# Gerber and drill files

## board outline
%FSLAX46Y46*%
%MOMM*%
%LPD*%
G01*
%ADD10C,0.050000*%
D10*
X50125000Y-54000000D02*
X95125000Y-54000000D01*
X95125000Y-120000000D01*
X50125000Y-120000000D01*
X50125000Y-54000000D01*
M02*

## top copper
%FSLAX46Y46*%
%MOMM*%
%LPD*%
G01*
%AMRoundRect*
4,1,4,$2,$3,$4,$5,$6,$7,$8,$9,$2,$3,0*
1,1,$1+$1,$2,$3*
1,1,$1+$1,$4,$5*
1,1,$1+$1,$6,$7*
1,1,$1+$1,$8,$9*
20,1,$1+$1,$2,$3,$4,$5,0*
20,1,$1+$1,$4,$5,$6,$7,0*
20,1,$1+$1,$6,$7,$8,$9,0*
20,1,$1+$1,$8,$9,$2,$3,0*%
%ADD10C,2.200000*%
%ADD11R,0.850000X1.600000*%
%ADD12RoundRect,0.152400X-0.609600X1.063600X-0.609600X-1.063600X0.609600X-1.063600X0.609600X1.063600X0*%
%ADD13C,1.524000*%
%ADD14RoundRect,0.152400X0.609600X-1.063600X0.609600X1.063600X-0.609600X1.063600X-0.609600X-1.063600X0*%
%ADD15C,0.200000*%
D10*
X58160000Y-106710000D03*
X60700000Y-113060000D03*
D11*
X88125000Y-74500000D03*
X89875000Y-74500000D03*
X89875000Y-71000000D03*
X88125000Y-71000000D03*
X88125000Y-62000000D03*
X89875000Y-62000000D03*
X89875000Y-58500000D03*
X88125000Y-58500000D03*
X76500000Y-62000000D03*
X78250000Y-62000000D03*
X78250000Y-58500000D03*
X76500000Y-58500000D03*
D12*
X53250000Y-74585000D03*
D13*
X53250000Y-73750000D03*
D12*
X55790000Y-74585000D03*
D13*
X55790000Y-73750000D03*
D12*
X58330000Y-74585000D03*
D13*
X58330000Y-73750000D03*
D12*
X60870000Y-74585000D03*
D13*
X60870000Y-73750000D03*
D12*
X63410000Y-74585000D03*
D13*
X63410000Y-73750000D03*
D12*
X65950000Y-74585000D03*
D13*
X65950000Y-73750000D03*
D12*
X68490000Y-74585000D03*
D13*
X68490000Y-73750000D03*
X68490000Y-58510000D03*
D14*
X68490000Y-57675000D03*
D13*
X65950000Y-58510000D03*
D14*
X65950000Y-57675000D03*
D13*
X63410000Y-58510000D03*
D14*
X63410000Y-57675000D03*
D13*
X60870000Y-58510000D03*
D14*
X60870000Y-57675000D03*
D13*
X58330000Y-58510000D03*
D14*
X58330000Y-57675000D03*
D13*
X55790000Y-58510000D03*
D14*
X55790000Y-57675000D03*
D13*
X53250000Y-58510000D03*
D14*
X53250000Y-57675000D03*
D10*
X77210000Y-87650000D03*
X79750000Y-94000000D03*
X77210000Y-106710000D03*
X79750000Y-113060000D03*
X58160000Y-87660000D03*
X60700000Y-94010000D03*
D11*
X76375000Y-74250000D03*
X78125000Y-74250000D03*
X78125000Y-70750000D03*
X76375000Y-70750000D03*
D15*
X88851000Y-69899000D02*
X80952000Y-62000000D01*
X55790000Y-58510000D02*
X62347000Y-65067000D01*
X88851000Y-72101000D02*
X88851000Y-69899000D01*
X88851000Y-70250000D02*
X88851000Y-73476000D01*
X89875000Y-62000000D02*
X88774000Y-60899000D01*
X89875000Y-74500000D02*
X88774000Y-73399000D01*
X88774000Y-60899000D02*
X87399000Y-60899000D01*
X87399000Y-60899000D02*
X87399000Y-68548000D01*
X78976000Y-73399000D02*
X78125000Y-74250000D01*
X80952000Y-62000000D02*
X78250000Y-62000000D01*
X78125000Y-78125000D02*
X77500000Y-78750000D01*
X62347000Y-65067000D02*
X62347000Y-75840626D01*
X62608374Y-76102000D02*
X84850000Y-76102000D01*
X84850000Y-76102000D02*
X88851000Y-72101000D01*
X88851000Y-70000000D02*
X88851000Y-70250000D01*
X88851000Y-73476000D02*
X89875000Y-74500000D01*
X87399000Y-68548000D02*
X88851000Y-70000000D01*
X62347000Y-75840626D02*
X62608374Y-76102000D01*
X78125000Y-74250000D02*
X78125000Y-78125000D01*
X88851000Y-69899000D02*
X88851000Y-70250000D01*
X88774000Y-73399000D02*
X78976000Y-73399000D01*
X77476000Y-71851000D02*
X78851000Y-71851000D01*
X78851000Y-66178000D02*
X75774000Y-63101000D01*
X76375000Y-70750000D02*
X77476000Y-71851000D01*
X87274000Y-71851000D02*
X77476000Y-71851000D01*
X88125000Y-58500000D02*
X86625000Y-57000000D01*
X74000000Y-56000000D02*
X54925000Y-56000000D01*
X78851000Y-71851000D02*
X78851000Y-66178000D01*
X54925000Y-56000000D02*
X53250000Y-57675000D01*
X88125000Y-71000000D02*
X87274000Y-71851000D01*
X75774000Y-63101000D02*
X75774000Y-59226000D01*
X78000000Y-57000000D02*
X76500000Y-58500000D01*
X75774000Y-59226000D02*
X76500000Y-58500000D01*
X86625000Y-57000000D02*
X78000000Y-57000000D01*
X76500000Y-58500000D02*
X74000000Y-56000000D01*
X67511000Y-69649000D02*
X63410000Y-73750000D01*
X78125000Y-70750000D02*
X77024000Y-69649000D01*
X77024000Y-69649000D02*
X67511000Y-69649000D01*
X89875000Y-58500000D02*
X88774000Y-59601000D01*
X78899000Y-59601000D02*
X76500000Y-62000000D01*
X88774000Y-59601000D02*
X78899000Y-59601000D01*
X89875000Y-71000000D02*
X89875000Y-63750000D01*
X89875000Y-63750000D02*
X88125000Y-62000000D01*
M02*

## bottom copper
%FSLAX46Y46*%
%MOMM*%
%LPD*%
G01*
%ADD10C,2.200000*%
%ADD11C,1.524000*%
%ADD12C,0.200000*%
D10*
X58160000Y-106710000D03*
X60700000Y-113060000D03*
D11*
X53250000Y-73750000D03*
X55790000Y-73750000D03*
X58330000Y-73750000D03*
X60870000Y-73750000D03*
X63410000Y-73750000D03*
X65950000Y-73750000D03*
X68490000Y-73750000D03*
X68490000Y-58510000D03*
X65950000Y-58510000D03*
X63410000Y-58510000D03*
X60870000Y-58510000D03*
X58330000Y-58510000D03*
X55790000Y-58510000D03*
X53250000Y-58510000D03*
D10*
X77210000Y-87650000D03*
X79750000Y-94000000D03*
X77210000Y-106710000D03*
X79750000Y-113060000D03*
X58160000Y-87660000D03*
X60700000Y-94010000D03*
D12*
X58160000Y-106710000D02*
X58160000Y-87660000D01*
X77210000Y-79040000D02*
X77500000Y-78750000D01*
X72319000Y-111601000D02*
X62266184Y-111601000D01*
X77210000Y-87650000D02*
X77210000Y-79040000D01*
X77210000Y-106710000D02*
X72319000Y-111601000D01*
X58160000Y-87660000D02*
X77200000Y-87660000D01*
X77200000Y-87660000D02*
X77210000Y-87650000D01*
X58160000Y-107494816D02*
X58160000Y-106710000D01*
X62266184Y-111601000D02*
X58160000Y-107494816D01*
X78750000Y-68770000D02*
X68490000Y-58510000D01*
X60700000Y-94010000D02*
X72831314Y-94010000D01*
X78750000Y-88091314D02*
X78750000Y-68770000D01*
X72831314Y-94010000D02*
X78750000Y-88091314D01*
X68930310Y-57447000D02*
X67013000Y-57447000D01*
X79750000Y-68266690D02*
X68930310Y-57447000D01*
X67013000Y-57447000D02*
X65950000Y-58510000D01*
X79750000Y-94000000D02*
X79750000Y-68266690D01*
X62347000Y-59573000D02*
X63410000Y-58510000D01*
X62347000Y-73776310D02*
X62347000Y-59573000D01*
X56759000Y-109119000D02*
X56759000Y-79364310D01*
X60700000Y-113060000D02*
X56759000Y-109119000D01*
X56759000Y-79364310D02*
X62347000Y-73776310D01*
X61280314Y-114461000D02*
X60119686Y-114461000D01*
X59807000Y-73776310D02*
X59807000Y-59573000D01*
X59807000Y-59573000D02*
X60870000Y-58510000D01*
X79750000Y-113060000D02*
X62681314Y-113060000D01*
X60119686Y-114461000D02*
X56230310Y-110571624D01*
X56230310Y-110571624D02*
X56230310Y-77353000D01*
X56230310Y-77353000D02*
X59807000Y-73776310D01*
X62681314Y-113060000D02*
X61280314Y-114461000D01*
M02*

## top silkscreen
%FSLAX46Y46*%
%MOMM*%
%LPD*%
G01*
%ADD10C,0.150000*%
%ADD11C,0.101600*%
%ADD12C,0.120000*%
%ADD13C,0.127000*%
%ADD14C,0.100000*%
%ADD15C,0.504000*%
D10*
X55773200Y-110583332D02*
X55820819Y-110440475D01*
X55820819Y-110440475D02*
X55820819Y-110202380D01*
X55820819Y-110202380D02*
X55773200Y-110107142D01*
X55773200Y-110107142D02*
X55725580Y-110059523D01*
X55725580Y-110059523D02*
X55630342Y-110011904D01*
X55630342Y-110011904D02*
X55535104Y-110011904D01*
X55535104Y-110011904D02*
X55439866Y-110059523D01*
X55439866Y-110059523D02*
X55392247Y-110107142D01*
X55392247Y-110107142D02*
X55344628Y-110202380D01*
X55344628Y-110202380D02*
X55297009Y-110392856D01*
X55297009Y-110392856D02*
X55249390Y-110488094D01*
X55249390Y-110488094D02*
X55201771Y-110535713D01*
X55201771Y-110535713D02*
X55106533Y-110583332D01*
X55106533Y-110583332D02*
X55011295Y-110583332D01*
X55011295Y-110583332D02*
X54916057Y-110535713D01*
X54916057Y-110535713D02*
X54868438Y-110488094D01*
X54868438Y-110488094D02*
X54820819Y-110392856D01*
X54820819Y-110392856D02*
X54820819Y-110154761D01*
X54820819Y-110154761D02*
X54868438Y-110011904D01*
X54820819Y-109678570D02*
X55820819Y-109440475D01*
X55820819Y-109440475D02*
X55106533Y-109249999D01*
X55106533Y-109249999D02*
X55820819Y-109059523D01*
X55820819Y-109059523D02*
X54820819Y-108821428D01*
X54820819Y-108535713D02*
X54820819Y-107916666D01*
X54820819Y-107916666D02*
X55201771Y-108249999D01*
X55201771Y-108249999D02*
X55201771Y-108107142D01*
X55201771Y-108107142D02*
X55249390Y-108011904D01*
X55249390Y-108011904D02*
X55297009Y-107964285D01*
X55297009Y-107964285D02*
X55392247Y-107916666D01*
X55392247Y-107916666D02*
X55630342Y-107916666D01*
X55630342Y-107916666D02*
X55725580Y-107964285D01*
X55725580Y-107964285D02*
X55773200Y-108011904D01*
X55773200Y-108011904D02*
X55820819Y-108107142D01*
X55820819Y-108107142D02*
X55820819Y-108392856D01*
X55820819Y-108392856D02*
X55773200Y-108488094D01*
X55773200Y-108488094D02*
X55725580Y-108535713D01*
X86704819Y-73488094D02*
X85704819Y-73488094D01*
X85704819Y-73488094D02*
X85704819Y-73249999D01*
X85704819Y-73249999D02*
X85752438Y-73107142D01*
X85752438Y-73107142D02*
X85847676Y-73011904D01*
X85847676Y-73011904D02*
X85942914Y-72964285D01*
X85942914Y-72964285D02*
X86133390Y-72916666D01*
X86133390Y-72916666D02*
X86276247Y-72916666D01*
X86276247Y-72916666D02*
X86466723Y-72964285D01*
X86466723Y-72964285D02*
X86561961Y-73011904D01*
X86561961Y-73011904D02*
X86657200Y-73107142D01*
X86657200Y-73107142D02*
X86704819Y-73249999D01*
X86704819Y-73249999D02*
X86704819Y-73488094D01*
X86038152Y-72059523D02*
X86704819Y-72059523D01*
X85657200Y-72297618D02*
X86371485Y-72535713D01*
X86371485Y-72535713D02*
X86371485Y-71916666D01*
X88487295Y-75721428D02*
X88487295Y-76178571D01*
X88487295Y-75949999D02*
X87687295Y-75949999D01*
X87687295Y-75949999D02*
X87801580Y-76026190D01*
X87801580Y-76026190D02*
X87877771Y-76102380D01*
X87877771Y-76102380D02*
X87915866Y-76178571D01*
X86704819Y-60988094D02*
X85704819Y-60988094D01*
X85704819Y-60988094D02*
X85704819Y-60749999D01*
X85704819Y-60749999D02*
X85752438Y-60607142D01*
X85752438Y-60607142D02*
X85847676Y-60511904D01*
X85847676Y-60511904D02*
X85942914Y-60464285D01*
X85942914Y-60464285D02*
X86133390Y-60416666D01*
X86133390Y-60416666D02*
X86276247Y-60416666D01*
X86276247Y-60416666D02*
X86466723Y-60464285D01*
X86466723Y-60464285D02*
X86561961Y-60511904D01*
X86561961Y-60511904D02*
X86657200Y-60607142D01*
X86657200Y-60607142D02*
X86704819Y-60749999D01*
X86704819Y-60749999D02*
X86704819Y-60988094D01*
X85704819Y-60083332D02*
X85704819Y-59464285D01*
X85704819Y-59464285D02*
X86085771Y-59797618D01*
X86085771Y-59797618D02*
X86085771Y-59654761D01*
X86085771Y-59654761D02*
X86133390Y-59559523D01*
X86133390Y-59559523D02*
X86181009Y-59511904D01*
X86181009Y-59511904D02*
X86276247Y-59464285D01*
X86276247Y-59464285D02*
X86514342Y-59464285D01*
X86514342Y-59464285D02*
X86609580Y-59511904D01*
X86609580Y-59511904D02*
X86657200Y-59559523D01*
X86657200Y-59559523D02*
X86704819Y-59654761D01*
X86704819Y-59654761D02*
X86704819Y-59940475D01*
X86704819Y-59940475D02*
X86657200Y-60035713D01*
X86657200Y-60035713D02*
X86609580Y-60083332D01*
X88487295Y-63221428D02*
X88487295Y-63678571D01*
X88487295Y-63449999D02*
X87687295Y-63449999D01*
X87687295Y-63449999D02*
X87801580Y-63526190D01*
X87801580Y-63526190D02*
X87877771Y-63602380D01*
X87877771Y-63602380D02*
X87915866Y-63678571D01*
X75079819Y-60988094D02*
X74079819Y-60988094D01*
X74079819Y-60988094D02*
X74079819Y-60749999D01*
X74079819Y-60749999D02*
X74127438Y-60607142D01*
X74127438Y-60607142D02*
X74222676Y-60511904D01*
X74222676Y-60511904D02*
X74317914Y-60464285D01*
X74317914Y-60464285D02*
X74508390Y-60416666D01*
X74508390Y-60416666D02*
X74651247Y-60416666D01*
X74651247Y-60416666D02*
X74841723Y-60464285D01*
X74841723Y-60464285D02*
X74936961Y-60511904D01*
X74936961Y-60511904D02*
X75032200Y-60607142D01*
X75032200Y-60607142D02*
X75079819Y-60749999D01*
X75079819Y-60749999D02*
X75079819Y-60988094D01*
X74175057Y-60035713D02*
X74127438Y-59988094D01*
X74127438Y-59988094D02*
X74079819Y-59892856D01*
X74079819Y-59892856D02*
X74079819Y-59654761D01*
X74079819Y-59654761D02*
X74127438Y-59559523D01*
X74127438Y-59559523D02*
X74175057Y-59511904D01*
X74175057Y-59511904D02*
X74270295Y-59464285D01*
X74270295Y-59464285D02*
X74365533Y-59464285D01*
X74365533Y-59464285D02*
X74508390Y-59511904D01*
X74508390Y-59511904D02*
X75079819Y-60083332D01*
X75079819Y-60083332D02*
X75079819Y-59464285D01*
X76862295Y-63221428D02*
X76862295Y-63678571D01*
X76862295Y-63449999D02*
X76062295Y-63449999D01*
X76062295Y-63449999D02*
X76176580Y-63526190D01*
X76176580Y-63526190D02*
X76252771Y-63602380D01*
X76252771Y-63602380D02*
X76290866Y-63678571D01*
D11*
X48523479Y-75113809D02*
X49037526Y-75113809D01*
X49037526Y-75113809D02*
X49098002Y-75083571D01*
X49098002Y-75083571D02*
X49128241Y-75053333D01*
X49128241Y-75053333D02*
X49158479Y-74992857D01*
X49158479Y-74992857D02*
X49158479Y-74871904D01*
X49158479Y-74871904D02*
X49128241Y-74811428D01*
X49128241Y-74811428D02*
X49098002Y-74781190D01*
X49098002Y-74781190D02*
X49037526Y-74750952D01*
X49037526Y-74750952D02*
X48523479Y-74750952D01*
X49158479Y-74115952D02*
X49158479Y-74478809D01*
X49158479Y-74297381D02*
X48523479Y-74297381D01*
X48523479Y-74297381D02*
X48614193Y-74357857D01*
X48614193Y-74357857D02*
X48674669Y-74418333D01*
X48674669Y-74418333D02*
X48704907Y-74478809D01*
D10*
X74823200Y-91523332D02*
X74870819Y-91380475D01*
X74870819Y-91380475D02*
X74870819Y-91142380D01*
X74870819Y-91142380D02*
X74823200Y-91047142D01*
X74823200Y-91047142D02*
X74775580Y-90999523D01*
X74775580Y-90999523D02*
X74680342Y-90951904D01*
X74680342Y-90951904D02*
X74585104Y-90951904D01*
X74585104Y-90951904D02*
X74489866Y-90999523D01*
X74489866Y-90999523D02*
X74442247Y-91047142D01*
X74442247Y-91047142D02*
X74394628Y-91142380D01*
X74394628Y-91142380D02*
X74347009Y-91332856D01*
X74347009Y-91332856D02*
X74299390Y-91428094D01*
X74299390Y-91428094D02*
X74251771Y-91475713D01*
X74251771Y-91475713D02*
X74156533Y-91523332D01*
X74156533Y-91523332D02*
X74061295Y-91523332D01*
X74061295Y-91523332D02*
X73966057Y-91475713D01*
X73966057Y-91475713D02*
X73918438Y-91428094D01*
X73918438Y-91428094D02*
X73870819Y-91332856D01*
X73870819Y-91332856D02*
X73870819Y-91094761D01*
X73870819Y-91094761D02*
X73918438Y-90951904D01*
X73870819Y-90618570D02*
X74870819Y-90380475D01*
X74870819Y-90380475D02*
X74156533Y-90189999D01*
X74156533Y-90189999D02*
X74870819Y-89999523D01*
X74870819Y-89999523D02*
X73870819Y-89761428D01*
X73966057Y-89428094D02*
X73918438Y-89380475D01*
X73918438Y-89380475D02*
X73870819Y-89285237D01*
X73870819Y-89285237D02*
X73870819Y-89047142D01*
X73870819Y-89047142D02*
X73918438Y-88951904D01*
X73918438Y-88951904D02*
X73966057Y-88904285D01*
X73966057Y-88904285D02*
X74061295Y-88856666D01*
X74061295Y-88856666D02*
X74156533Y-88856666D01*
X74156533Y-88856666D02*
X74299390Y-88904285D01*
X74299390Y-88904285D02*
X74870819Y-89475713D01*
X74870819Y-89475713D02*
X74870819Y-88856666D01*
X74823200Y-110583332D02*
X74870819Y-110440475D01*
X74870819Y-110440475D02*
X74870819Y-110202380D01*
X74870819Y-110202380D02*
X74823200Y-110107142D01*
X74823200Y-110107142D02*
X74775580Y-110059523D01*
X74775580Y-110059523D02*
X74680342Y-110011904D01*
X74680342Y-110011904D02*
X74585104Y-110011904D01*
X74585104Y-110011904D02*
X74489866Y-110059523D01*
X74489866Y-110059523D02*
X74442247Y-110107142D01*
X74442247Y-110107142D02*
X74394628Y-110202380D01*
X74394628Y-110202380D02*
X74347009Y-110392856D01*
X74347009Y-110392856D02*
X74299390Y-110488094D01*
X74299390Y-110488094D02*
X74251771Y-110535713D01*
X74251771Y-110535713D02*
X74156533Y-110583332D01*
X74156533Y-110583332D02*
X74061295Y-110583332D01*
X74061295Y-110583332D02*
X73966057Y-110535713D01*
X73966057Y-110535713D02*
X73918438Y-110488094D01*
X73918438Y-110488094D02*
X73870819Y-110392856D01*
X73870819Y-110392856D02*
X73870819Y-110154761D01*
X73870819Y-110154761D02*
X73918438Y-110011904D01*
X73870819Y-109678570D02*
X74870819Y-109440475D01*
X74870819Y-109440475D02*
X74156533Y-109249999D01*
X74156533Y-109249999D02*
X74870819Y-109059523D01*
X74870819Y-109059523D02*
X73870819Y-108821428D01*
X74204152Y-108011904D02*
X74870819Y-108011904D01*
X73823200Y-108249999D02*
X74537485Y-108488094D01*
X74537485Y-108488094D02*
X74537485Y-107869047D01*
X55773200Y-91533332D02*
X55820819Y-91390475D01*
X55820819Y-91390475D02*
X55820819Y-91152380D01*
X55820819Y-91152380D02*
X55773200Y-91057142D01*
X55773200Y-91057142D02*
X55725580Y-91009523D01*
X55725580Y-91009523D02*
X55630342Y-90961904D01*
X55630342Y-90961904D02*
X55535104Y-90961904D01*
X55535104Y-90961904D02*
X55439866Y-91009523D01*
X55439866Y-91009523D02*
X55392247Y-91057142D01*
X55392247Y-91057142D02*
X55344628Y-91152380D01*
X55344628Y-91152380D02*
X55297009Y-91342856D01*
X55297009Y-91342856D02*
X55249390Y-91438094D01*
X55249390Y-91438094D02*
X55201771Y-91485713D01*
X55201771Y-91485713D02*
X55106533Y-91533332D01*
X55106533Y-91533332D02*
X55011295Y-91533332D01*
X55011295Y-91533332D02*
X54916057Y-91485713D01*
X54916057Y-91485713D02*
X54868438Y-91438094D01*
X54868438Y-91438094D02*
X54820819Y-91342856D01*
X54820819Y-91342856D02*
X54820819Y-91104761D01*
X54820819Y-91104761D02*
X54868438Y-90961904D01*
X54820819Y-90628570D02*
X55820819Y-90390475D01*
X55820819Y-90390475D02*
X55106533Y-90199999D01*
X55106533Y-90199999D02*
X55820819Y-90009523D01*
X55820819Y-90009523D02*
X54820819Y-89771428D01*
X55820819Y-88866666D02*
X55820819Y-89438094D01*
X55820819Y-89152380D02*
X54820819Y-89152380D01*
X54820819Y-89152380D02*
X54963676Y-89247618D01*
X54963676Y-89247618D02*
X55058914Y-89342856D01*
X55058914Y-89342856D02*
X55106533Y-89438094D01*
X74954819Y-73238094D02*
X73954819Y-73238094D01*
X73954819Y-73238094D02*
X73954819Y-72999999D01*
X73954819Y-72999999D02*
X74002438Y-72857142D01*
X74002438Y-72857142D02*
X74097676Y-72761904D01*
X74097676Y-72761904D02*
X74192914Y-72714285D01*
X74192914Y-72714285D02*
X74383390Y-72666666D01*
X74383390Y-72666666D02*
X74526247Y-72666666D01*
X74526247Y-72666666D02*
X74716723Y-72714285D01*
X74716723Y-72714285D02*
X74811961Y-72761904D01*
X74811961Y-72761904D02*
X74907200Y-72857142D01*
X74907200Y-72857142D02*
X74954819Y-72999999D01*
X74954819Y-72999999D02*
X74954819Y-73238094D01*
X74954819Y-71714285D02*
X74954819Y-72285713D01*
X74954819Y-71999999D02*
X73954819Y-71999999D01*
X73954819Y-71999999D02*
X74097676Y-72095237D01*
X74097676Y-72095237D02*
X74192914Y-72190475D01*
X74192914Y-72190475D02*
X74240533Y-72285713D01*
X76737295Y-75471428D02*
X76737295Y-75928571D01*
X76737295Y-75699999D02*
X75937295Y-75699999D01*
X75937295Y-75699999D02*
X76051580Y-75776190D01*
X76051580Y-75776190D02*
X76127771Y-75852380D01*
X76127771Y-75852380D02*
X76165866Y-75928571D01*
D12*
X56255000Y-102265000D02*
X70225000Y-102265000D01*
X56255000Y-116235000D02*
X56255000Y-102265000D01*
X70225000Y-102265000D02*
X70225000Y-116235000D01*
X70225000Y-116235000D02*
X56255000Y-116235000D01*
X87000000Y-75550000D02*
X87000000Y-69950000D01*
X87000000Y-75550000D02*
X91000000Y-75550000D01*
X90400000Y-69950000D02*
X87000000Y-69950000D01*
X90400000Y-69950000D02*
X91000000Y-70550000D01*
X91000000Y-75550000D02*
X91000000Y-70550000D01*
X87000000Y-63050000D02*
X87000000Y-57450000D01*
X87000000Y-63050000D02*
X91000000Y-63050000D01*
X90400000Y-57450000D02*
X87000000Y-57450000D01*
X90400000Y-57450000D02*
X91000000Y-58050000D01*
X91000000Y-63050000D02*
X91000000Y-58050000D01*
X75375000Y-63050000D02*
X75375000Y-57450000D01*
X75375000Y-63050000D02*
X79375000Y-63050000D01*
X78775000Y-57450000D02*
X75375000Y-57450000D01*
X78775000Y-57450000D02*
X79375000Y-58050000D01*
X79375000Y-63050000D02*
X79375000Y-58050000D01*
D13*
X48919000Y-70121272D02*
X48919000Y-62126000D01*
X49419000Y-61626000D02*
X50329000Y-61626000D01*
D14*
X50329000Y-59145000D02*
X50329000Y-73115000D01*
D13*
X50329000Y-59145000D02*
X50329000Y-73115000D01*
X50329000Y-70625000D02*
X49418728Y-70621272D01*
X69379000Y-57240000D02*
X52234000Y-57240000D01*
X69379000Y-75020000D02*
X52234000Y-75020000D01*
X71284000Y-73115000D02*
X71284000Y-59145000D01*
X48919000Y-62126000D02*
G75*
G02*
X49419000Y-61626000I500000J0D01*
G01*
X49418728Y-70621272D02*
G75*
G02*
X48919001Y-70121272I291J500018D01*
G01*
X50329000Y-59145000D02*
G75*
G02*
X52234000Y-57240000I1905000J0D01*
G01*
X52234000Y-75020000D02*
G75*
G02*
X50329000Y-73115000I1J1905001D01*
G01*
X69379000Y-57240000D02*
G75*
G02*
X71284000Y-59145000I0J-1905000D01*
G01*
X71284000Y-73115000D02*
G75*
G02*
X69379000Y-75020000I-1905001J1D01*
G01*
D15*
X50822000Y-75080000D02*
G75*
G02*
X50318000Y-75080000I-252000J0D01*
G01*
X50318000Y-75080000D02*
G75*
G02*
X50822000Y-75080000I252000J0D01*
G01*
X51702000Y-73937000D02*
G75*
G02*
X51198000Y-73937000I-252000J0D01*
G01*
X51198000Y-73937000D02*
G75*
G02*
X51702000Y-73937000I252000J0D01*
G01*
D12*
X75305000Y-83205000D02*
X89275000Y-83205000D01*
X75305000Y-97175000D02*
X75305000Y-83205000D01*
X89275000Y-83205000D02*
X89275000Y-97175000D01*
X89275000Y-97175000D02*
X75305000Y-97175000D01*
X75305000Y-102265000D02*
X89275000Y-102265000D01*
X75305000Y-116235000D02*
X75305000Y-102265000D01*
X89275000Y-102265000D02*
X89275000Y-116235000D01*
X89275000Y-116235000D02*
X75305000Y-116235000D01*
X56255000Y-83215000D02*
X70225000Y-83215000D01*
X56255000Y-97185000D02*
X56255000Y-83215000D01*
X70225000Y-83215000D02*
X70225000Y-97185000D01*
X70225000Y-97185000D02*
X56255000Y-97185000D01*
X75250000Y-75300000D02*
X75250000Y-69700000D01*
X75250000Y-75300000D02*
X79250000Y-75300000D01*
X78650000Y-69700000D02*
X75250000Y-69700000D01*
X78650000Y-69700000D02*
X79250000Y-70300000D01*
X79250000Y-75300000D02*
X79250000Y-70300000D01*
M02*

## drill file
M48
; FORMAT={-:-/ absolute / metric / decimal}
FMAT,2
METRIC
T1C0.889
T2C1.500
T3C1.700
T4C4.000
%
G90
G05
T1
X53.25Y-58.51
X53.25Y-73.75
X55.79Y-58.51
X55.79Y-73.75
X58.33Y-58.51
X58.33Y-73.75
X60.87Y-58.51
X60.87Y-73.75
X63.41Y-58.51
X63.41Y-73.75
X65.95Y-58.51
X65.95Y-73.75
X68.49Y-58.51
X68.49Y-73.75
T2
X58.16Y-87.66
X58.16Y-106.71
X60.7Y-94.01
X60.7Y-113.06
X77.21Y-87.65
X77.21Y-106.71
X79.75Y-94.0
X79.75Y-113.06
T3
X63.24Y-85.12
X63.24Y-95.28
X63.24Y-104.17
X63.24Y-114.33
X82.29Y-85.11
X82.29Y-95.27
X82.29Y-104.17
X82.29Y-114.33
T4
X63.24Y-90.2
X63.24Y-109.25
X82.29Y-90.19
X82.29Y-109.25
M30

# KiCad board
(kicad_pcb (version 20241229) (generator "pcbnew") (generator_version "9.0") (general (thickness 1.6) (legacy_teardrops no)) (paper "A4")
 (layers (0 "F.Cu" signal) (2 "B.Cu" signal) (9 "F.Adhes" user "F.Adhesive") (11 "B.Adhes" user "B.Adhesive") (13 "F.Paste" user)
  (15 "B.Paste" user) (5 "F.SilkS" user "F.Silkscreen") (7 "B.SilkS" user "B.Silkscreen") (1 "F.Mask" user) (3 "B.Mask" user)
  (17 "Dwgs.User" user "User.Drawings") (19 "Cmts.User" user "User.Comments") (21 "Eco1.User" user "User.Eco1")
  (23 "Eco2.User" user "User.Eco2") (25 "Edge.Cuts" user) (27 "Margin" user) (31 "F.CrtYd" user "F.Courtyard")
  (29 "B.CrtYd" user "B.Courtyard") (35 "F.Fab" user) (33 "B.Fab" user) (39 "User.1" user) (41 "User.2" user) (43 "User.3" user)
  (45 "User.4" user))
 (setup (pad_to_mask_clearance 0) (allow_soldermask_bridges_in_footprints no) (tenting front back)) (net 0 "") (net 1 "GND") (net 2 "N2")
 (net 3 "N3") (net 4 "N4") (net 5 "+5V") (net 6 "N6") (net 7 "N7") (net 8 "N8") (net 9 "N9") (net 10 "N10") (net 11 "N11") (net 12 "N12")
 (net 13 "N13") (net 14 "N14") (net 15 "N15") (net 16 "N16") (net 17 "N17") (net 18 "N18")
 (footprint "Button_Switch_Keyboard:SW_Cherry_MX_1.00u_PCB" (layer "F.Cu") (at 58.16 106.71 90)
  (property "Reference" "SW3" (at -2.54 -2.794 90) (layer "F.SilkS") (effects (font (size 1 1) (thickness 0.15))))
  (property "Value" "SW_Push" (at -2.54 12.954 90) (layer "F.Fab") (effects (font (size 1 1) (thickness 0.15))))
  (fp_line (start 4.445 -1.905) (end 4.445 12.065) (stroke (width 0.12) (type solid)) (layer "F.SilkS"))
  (fp_line (start -9.525 -1.905) (end 4.445 -1.905) (stroke (width 0.12) (type solid)) (layer "F.SilkS"))
  (fp_line (start 4.445 12.065) (end -9.525 12.065) (stroke (width 0.12) (type solid)) (layer "F.SilkS"))
  (fp_line (start -9.525 12.065) (end -9.525 -1.905) (stroke (width 0.12) (type solid)) (layer "F.SilkS"))
  (pad "" np_thru_hole circle (at -7.62 5.08 90) (size 1.7 1.7) (drill 1.7) (layers "*.Cu" "*.Mask"))
  (pad "" np_thru_hole circle (at -2.54 5.08 90) (size 4 4) (drill 4) (layers "*.Cu" "*.Mask"))
  (pad "" np_thru_hole circle (at 2.54 5.08 90) (size 1.7 1.7) (drill 1.7) (layers "*.Cu" "*.Mask"))
  (pad "1" thru_hole circle (at 0 0 90) (size 2.2 2.2) (drill 1.5) (layers "*.Cu" "*.Mask") (remove_unused_layers no) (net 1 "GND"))
  (pad "2" thru_hole circle (at -6.35 2.54 90) (size 2.2 2.2) (drill 1.5) (layers "*.Cu" "*.Mask") (remove_unused_layers no) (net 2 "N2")))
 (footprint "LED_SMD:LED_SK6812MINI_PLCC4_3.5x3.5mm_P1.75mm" (layer "F.Cu") (at 89 72.75 90)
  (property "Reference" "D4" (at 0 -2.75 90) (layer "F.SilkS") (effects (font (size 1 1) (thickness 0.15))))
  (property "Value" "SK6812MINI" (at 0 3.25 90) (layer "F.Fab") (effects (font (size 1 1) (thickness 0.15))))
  (fp_line (start -2.8 -2) (end 2.8 -2) (stroke (width 0.12) (type solid)) (layer "F.SilkS"))
  (fp_line (start -2.8 -2) (end -2.8 2) (stroke (width 0.12) (type default)) (layer "F.SilkS"))
  (fp_line (start 2.8 1.4) (end 2.8 -2) (stroke (width 0.12) (type solid)) (layer "F.SilkS"))
  (fp_line (start 2.8 1.4) (end 2.2 2) (stroke (width 0.12) (type default)) (layer "F.SilkS"))
  (fp_line (start -2.8 2) (end 2.2 2) (stroke (width 0.12) (type solid)) (layer "F.SilkS"))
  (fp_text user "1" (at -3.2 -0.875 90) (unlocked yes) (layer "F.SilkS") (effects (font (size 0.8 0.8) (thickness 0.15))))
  (pad "1" smd rect (at -1.75 -0.875 90) (size 1.6 0.85) (layers "F.Cu" "F.Mask" "F.Paste") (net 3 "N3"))
  (pad "2" smd rect (at -1.75 0.875 90) (size 1.6 0.85) (layers "F.Cu" "F.Mask" "F.Paste") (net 1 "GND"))
  (pad "3" smd rect (at 1.75 0.875 90) (size 1.6 0.85) (layers "F.Cu" "F.Mask" "F.Paste") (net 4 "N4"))
  (pad "4" smd rect (at 1.75 -0.875 90) (size 1.6 0.85) (layers "F.Cu" "F.Mask" "F.Paste") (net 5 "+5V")))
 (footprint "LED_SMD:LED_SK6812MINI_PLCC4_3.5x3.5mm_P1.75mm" (layer "F.Cu") (at 89 60.25 90)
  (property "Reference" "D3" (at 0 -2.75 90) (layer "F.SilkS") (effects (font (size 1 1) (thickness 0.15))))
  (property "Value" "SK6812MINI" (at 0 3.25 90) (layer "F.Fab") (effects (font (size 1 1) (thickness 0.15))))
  (fp_line (start -2.8 -2) (end 2.8 -2) (stroke (width 0.12) (type solid)) (layer "F.SilkS"))
  (fp_line (start -2.8 -2) (end -2.8 2) (stroke (width 0.12) (type default)) (layer "F.SilkS"))
  (fp_line (start 2.8 1.4) (end 2.8 -2) (stroke (width 0.12) (type solid)) (layer "F.SilkS"))
  (fp_line (start 2.8 1.4) (end 2.2 2) (stroke (width 0.12) (type default)) (layer "F.SilkS"))
  (fp_line (start -2.8 2) (end 2.2 2) (stroke (width 0.12) (type solid)) (layer "F.SilkS"))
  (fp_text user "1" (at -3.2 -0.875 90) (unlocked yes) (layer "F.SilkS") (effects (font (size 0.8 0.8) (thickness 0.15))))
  (pad "1" smd rect (at -1.75 -0.875 90) (size 1.6 0.85) (layers "F.Cu" "F.Mask" "F.Paste") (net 4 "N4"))
  (pad "2" smd rect (at -1.75 0.875 90) (size 1.6 0.85) (layers "F.Cu" "F.Mask" "F.Paste") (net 1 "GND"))
  (pad "3" smd rect (at 1.75 0.875 90) (size 1.6 0.85) (layers "F.Cu" "F.Mask" "F.Paste") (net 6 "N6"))
  (pad "4" smd rect (at 1.75 -0.875 90) (size 1.6 0.85) (layers "F.Cu" "F.Mask" "F.Paste") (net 5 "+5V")))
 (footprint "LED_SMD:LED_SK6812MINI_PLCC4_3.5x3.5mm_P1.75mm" (layer "F.Cu") (at 77.375 60.25 90)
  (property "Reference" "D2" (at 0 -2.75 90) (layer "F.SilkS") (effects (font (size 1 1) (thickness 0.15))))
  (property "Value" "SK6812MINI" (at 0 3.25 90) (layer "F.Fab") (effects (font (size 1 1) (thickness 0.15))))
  (fp_line (start -2.8 -2) (end 2.8 -2) (stroke (width 0.12) (type solid)) (layer "F.SilkS"))
  (fp_line (start -2.8 -2) (end -2.8 2) (stroke (width 0.12) (type default)) (layer "F.SilkS"))
  (fp_line (start 2.8 1.4) (end 2.8 -2) (stroke (width 0.12) (type solid)) (layer "F.SilkS"))
  (fp_line (start 2.8 1.4) (end 2.2 2) (stroke (width 0.12) (type default)) (layer "F.SilkS"))
  (fp_line (start -2.8 2) (end 2.2 2) (stroke (width 0.12) (type solid)) (layer "F.SilkS"))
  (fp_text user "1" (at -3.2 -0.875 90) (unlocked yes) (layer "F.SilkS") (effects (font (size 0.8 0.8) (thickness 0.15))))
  (pad "1" smd rect (at -1.75 -0.875 90) (size 1.6 0.85) (layers "F.Cu" "F.Mask" "F.Paste") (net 6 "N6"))
  (pad "2" smd rect (at -1.75 0.875 90) (size 1.6 0.85) (layers "F.Cu" "F.Mask" "F.Paste") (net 1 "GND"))
  (pad "3" smd rect (at 1.75 0.875 90) (size 1.6 0.85) (layers "F.Cu" "F.Mask" "F.Paste") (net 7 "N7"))
  (pad "4" smd rect (at 1.75 -0.875 90) (size 1.6 0.85) (layers "F.Cu" "F.Mask" "F.Paste") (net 5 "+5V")))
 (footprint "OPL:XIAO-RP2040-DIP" (layer "F.Cu") (at 60.87 66.13 90)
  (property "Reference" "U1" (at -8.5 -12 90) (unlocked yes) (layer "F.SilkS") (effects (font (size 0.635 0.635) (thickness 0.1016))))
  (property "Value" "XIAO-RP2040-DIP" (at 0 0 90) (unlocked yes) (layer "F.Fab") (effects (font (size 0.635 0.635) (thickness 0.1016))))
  (fp_line (start -3.991272 -11.951) (end 4.004 -11.951) (stroke (width 0.127) (type solid)) (layer "F.SilkS"))
  (fp_line (start 4.504 -11.451) (end 4.504 -10.541) (stroke (width 0.127) (type solid)) (layer "F.SilkS"))
  (fp_line (start 6.985 -10.541) (end -6.985 -10.541) (stroke (width 0.1) (type solid)) (layer "F.SilkS"))
  (fp_line (start 6.985 -10.541) (end -6.985 -10.541) (stroke (width 0.127) (type solid)) (layer "F.SilkS"))
  (fp_line (start -4.495 -10.541) (end -4.491272 -11.451272) (stroke (width 0.127) (type solid)) (layer "F.SilkS"))
  (fp_line (start 8.89 8.509) (end 8.89 -8.636) (stroke (width 0.127) (type solid)) (layer "F.SilkS"))
  (fp_line (start -8.89 8.509) (end -8.89 -8.636) (stroke (width 0.127) (type solid)) (layer "F.SilkS"))
  (fp_line (start -6.985 10.414) (end 6.985 10.414) (stroke (width 0.127) (type solid)) (layer "F.SilkS"))
  (fp_arc (start 4.004 -11.951) (mid 4.357553 -11.804553) (end 4.504 -11.451) (stroke (width 0.127) (type default)) (layer "F.SilkS"))
  (fp_arc (start -4.491272 -11.451272) (mid -4.344728 -11.80464) (end -3.991272 -11.951) (stroke (width 0.127) (type default))
   (layer "F.SilkS"))
  (fp_arc (start 6.985 -10.541) (mid 8.332038 -9.983038) (end 8.89 -8.636) (stroke (width 0.127) (type solid)) (layer "F.SilkS"))
  (fp_arc (start -8.89 -8.636) (mid -8.332038 -9.983038) (end -6.985 -10.541) (stroke (width 0.127) (type solid)) (layer "F.SilkS"))
  (fp_arc (start 8.89 8.509) (mid 8.332038 9.856038) (end 6.985 10.414) (stroke (width 0.127) (type solid)) (layer "F.SilkS"))
  (fp_arc (start -6.985 10.414) (mid -8.332038 9.856038) (end -8.89 8.509) (stroke (width 0.127) (type solid)) (layer "F.SilkS"))
  (fp_circle (center -8.95 -10.3) (end -8.95 -10.554) (stroke (width 0.5) (type solid)) (fill yes) (layer "F.SilkS"))
  (fp_circle (center -7.807 -9.42) (end -7.807 -9.674) (stroke (width 0.5) (type solid)) (fill yes) (layer "F.SilkS"))
  (pad "1" smd roundrect (at -8.455 -7.62 270) (size 2.432 1.524) (layers "F.Cu" "F.Mask") (roundrect_rratio 0.1) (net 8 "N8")
   (thermal_bridge_angle 45))
  (pad "1" thru_hole circle (at -7.62 -7.62 270) (size 1.524 1.524) (drill 0.889) (layers "*.Cu" "*.Mask") (remove_unused_layers no)
   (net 8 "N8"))
  (pad "2" smd roundrect (at -8.455 -5.08 270) (size 2.432 1.524) (layers "F.Cu" "F.Mask") (roundrect_rratio 0.1) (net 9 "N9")
   (thermal_bridge_angle 45))
  (pad "2" thru_hole circle (at -7.62 -5.08 270) (size 1.524 1.524) (drill 0.889) (layers "*.Cu" "*.Mask") (remove_unused_layers no)
   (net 9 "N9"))
  (pad "3" smd roundrect (at -8.455 -2.54 270) (size 2.432 1.524) (layers "F.Cu" "F.Mask") (roundrect_rratio 0.1) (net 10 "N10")
   (thermal_bridge_angle 45))
  (pad "3" thru_hole circle (at -7.62 -2.54 270) (size 1.524 1.524) (drill 0.889) (layers "*.Cu" "*.Mask") (remove_unused_layers no)
   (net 10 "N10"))
  (pad "4" smd roundrect (at -8.455 0 270) (size 2.432 1.524) (layers "F.Cu" "F.Mask") (roundrect_rratio 0.1) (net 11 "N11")
   (thermal_bridge_angle 45))
  (pad "4" thru_hole circle (at -7.62 0 270) (size 1.524 1.524) (drill 0.889) (layers "*.Cu" "*.Mask") (remove_unused_layers no)
   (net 11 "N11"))
  (pad "5" smd roundrect (at -8.455 2.54 270) (size 2.432 1.524) (layers "F.Cu" "F.Mask") (roundrect_rratio 0.1) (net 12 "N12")
   (thermal_bridge_angle 45))
  (pad "5" thru_hole circle (at -7.62 2.54 270) (size 1.524 1.524) (drill 0.889) (layers "*.Cu" "*.Mask") (remove_unused_layers no)
   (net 12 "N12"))
  (pad "6" smd roundrect (at -8.455 5.08 270) (size 2.432 1.524) (layers "F.Cu" "F.Mask") (roundrect_rratio 0.1) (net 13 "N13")
   (thermal_bridge_angle 45))
  (pad "6" thru_hole circle (at -7.62 5.08 270) (size 1.524 1.524) (drill 0.889) (layers "*.Cu" "*.Mask") (remove_unused_layers no)
   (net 13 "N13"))
  (pad "7" smd roundrect (at -8.455 7.62 270) (size 2.432 1.524) (layers "F.Cu" "F.Mask") (roundrect_rratio 0.1) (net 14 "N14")
   (thermal_bridge_angle 45))
  (pad "7" thru_hole circle (at -7.62 7.62 270) (size 1.524 1.524) (drill 0.889) (layers "*.Cu" "*.Mask") (remove_unused_layers no)
   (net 14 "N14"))
  (pad "8" thru_hole circle (at 7.62 7.62 90) (size 1.524 1.524) (drill 0.889) (layers "*.Cu" "*.Mask") (remove_unused_layers no)
   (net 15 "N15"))
  (pad "8" smd roundrect (at 8.455 7.62 90) (size 2.432 1.524) (layers "F.Cu" "F.Mask") (roundrect_rratio 0.1) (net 15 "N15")
   (thermal_bridge_angle 45))
  (pad "9" thru_hole circle (at 7.62 5.08 90) (size 1.524 1.524) (drill 0.889) (layers "*.Cu" "*.Mask") (remove_unused_layers no)
   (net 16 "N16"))
  (pad "9" smd roundrect (at 8.455 5.08 90) (size 2.432 1.524) (layers "F.Cu" "F.Mask") (roundrect_rratio 0.1) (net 16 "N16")
   (thermal_bridge_angle 45))
  (pad "10" thru_hole circle (at 7.62 2.54 90) (size 1.524 1.524) (drill 0.889) (layers "*.Cu" "*.Mask") (remove_unused_layers no)
   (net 2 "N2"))
  (pad "10" smd roundrect (at 8.455 2.54 90) (size 2.432 1.524) (layers "F.Cu" "F.Mask") (roundrect_rratio 0.1) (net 2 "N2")
   (thermal_bridge_angle 45))
  (pad "11" thru_hole circle (at 7.62 0 90) (size 1.524 1.524) (drill 0.889) (layers "*.Cu" "*.Mask") (remove_unused_layers no)
   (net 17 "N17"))
  (pad "11" smd roundrect (at 8.455 0 90) (size 2.432 1.524) (layers "F.Cu" "F.Mask") (roundrect_rratio 0.1) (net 17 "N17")
   (thermal_bridge_angle 45))
  (pad "12" thru_hole circle (at 7.62 -2.54 90) (size 1.524 1.524) (drill 0.889) (layers "*.Cu" "*.Mask") (remove_unused_layers no)
   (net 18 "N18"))
  (pad "12" smd roundrect (at 8.455 -2.54 90) (size 2.432 1.524) (layers "F.Cu" "F.Mask") (roundrect_rratio 0.1) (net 18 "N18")
   (thermal_bridge_angle 45))
  (pad "13" thru_hole circle (at 7.62 -5.08 90) (size 1.524 1.524) (drill 0.889) (layers "*.Cu" "*.Mask") (remove_unused_layers no)
   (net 1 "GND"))
  (pad "13" smd roundrect (at 8.455 -5.08 90) (size 2.432 1.524) (layers "F.Cu" "F.Mask") (roundrect_rratio 0.1) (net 1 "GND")
   (thermal_bridge_angle 45))
  (pad "14" thru_hole circle (at 7.62 -7.62 90) (size 1.524 1.524) (drill 0.889) (layers "*.Cu" "*.Mask") (remove_unused_layers no)
   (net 5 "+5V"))
  (pad "14" smd roundrect (at 8.455 -7.62 90) (size 2.432 1.524) (layers "F.Cu" "F.Mask") (roundrect_rratio 0.1) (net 5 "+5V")
   (thermal_bridge_angle 45)))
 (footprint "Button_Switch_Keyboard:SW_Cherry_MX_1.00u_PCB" (layer "F.Cu") (at 77.21 87.65 90)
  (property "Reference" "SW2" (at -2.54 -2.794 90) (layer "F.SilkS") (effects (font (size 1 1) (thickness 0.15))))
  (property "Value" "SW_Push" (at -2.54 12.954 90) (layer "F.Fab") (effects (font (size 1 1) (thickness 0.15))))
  (fp_line (start 4.445 -1.905) (end 4.445 12.065) (stroke (width 0.12) (type solid)) (layer "F.SilkS"))
  (fp_line (start -9.525 -1.905) (end 4.445 -1.905) (stroke (width 0.12) (type solid)) (layer "F.SilkS"))
  (fp_line (start 4.445 12.065) (end -9.525 12.065) (stroke (width 0.12) (type solid)) (layer "F.SilkS"))
  (fp_line (start -9.525 12.065) (end -9.525 -1.905) (stroke (width 0.12) (type solid)) (layer "F.SilkS"))
  (pad "" np_thru_hole circle (at -7.62 5.08 90) (size 1.7 1.7) (drill 1.7) (layers "*.Cu" "*.Mask"))
  (pad "" np_thru_hole circle (at -2.54 5.08 90) (size 4 4) (drill 4) (layers "*.Cu" "*.Mask"))
  (pad "" np_thru_hole circle (at 2.54 5.08 90) (size 1.7 1.7) (drill 1.7) (layers "*.Cu" "*.Mask"))
  (pad "1" thru_hole circle (at 0 0 90) (size 2.2 2.2) (drill 1.5) (layers "*.Cu" "*.Mask") (remove_unused_layers no) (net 1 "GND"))
  (pad "2" thru_hole circle (at -6.35 2.54 90) (size 2.2 2.2) (drill 1.5) (layers "*.Cu" "*.Mask") (remove_unused_layers no) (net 16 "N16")))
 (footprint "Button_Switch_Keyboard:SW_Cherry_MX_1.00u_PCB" (layer "F.Cu") (at 77.21 106.71 90)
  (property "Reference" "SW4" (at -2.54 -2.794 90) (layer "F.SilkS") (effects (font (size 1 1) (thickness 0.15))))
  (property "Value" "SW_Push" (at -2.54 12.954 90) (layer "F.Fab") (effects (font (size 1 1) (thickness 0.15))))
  (fp_line (start 4.445 -1.905) (end 4.445 12.065) (stroke (width 0.12) (type solid)) (layer "F.SilkS"))
  (fp_line (start -9.525 -1.905) (end 4.445 -1.905) (stroke (width 0.12) (type solid)) (layer "F.SilkS"))
  (fp_line (start 4.445 12.065) (end -9.525 12.065) (stroke (width 0.12) (type solid)) (layer "F.SilkS"))
  (fp_line (start -9.525 12.065) (end -9.525 -1.905) (stroke (width 0.12) (type solid)) (layer "F.SilkS"))
  (pad "" np_thru_hole circle (at -7.62 5.08 90) (size 1.7 1.7) (drill 1.7) (layers "*.Cu" "*.Mask"))
  (pad "" np_thru_hole circle (at -2.54 5.08 90) (size 4 4) (drill 4) (layers "*.Cu" "*.Mask"))
  (pad "" np_thru_hole circle (at 2.54 5.08 90) (size 1.7 1.7) (drill 1.7) (layers "*.Cu" "*.Mask"))
  (pad "1" thru_hole circle (at 0 0 90) (size 2.2 2.2) (drill 1.5) (layers "*.Cu" "*.Mask") (remove_unused_layers no) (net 1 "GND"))
  (pad "2" thru_hole circle (at -6.35 2.54 90) (size 2.2 2.2) (drill 1.5) (layers "*.Cu" "*.Mask") (remove_unused_layers no) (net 17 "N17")))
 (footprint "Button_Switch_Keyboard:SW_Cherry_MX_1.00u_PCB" (layer "F.Cu") (at 58.16 87.66 90)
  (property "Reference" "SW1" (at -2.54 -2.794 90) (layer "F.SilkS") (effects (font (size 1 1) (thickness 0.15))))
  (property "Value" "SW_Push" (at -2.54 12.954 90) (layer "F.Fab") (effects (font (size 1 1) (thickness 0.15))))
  (fp_line (start 4.445 -1.905) (end 4.445 12.065) (stroke (width 0.12) (type solid)) (layer "F.SilkS"))
  (fp_line (start -9.525 -1.905) (end 4.445 -1.905) (stroke (width 0.12) (type solid)) (layer "F.SilkS"))
  (fp_line (start 4.445 12.065) (end -9.525 12.065) (stroke (width 0.12) (type solid)) (layer "F.SilkS"))
  (fp_line (start -9.525 12.065) (end -9.525 -1.905) (stroke (width 0.12) (type solid)) (layer "F.SilkS"))
  (pad "" np_thru_hole circle (at -7.62 5.08 90) (size 1.7 1.7) (drill 1.7) (layers "*.Cu" "*.Mask"))
  (pad "" np_thru_hole circle (at -2.54 5.08 90) (size 4 4) (drill 4) (layers "*.Cu" "*.Mask"))
  (pad "" np_thru_hole circle (at 2.54 5.08 90) (size 1.7 1.7) (drill 1.7) (layers "*.Cu" "*.Mask"))
  (pad "1" thru_hole circle (at 0 0 90) (size 2.2 2.2) (drill 1.5) (layers "*.Cu" "*.Mask") (remove_unused_layers no) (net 1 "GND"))
  (pad "2" thru_hole circle (at -6.35 2.54 90) (size 2.2 2.2) (drill 1.5) (layers "*.Cu" "*.Mask") (remove_unused_layers no) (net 15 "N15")))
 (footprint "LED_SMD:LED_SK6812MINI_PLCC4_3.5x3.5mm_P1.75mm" (layer "F.Cu") (at 77.25 72.5 90)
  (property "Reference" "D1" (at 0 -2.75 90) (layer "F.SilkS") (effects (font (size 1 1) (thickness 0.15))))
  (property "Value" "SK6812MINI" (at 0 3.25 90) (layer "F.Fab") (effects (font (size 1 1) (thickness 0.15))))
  (fp_line (start -2.8 -2) (end 2.8 -2) (stroke (width 0.12) (type solid)) (layer "F.SilkS"))
  (fp_line (start -2.8 -2) (end -2.8 2) (stroke (width 0.12) (type default)) (layer "F.SilkS"))
  (fp_line (start 2.8 1.4) (end 2.8 -2) (stroke (width 0.12) (type solid)) (layer "F.SilkS"))
  (fp_line (start 2.8 1.4) (end 2.2 2) (stroke (width 0.12) (type default)) (layer "F.SilkS"))
  (fp_line (start -2.8 2) (end 2.2 2) (stroke (width 0.12) (type solid)) (layer "F.SilkS"))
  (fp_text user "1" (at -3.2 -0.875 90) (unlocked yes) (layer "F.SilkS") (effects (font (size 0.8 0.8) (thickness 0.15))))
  (pad "1" smd rect (at -1.75 -0.875 90) (size 1.6 0.85) (layers "F.Cu" "F.Mask" "F.Paste") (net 7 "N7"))
  (pad "2" smd rect (at -1.75 0.875 90) (size 1.6 0.85) (layers "F.Cu" "F.Mask" "F.Paste") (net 1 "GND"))
  (pad "3" smd rect (at 1.75 0.875 90) (size 1.6 0.85) (layers "F.Cu" "F.Mask" "F.Paste") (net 12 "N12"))
  (pad "4" smd rect (at 1.75 -0.875 90) (size 1.6 0.85) (layers "F.Cu" "F.Mask" "F.Paste") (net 5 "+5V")))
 (gr_rect (start 50.125 54) (end 95.125 120) (stroke (width 0.05) (type default)) (fill no) (layer "Edge.Cuts"))
 (segment (start 88.851 69.899) (end 80.952 62) (width 0.2) (layer "F.Cu") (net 1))
 (segment (start 55.79 58.51) (end 62.347 65.067) (width 0.2) (layer "F.Cu") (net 1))
 (segment (start 88.851 72.101) (end 88.851 69.899) (width 0.2) (layer "F.Cu") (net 1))
 (segment (start 88.851 70.25) (end 88.851 73.476) (width 0.2) (layer "F.Cu") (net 1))
 (segment (start 89.875 62) (end 88.774 60.899) (width 0.2) (layer "F.Cu") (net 1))
 (segment (start 89.875 74.5) (end 88.774 73.399) (width 0.2) (layer "F.Cu") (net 1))
 (segment (start 88.774 60.899) (end 87.399 60.899) (width 0.2) (layer "F.Cu") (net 1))
 (segment (start 87.399 60.899) (end 87.399 68.548) (width 0.2) (layer "F.Cu") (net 1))
 (segment (start 78.976 73.399) (end 78.125 74.25) (width 0.2) (layer "F.Cu") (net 1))
 (segment (start 80.952 62) (end 78.25 62) (width 0.2) (layer "F.Cu") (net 1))
 (segment (start 78.125 78.125) (end 77.5 78.75) (width 0.2) (layer "F.Cu") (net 1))
 (segment (start 62.347 65.067) (end 62.347 75.840626) (width 0.2) (layer "F.Cu") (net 1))
 (segment (start 62.608374 76.102) (end 84.85 76.102) (width 0.2) (layer "F.Cu") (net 1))
 (segment (start 84.85 76.102) (end 88.851 72.101) (width 0.2) (layer "F.Cu") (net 1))
 (segment (start 88.851 70) (end 88.851 70.25) (width 0.2) (layer "F.Cu") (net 1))
 (segment (start 88.851 73.476) (end 89.875 74.5) (width 0.2) (layer "F.Cu") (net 1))
 (segment (start 87.399 68.548) (end 88.851 70) (width 0.2) (layer "F.Cu") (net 1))
 (segment (start 62.347 75.840626) (end 62.608374 76.102) (width 0.2) (layer "F.Cu") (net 1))
 (segment (start 78.125 74.25) (end 78.125 78.125) (width 0.2) (layer "F.Cu") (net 1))
 (segment (start 88.851 69.899) (end 88.851 70.25) (width 0.2) (layer "F.Cu") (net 1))
 (segment (start 88.774 73.399) (end 78.976 73.399) (width 0.2) (layer "F.Cu") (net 1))
 (segment (start 58.16 106.71) (end 58.16 87.66) (width 0.2) (layer "B.Cu") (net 1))
 (segment (start 77.21 79.04) (end 77.5 78.75) (width 0.2) (layer "B.Cu") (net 1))
 (segment (start 72.319 111.601) (end 62.266184 111.601) (width 0.2) (layer "B.Cu") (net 1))
 (segment (start 77.21 87.65) (end 77.21 79.04) (width 0.2) (layer "B.Cu") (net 1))
 (segment (start 77.21 106.71) (end 72.319 111.601) (width 0.2) (layer "B.Cu") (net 1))
 (segment (start 58.16 87.66) (end 77.2 87.66) (width 0.2) (layer "B.Cu") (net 1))
 (segment (start 77.2 87.66) (end 77.21 87.65) (width 0.2) (layer "B.Cu") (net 1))
 (segment (start 58.16 107.494816) (end 58.16 106.71) (width 0.2) (layer "B.Cu") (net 1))
 (segment (start 62.266184 111.601) (end 58.16 107.494816) (width 0.2) (layer "B.Cu") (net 1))
 (segment (start 77.476 71.851) (end 78.851 71.851) (width 0.2) (layer "F.Cu") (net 5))
 (segment (start 78.851 66.178) (end 75.774 63.101) (width 0.2) (layer "F.Cu") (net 5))
 (segment (start 76.375 70.75) (end 77.476 71.851) (width 0.2) (layer "F.Cu") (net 5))
 (segment (start 87.274 71.851) (end 77.476 71.851) (width 0.2) (layer "F.Cu") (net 5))
 (segment (start 88.125 58.5) (end 86.625 57) (width 0.2) (layer "F.Cu") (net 5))
 (segment (start 74 56) (end 54.925 56) (width 0.2) (layer "F.Cu") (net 5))
 (segment (start 78.851 71.851) (end 78.851 66.178) (width 0.2) (layer "F.Cu") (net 5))
 (segment (start 54.925 56) (end 53.25 57.675) (width 0.2) (layer "F.Cu") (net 5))
 (segment (start 88.125 71) (end 87.274 71.851) (width 0.2) (layer "F.Cu") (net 5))
 (segment (start 75.774 63.101) (end 75.774 59.226) (width 0.2) (layer "F.Cu") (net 5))
 (segment (start 78 57) (end 76.5 58.5) (width 0.2) (layer "F.Cu") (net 5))
 (segment (start 75.774 59.226) (end 76.5 58.5) (width 0.2) (layer "F.Cu") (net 5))
 (segment (start 86.625 57) (end 78 57) (width 0.2) (layer "F.Cu") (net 5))
 (segment (start 76.5 58.5) (end 74 56) (width 0.2) (layer "F.Cu") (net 5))
 (segment (start 67.511 69.649) (end 63.41 73.75) (width 0.2) (layer "F.Cu") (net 12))
 (segment (start 78.125 70.75) (end 77.024 69.649) (width 0.2) (layer "F.Cu") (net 12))
 (segment (start 77.024 69.649) (end 67.511 69.649) (width 0.2) (layer "F.Cu") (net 12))
 (segment (start 78.75 68.77) (end 68.49 58.51) (width 0.2) (layer "B.Cu") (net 15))
 (segment (start 60.7 94.01) (end 72.831314 94.01) (width 0.2) (layer "B.Cu") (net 15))
 (segment (start 78.75 88.091314) (end 78.75 68.77) (width 0.2) (layer "B.Cu") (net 15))
 (segment (start 72.831314 94.01) (end 78.75 88.091314) (width 0.2) (layer "B.Cu") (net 15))
 (segment (start 68.93031 57.447) (end 67.013 57.447) (width 0.2) (layer "B.Cu") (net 16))
 (segment (start 79.75 68.26669) (end 68.93031 57.447) (width 0.2) (layer "B.Cu") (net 16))
 (segment (start 67.013 57.447) (end 65.95 58.51) (width 0.2) (layer "B.Cu") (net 16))
 (segment (start 79.75 94) (end 79.75 68.26669) (width 0.2) (layer "B.Cu") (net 16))
 (segment (start 62.347 59.573) (end 63.41 58.51) (width 0.2) (layer "B.Cu") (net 2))
 (segment (start 62.347 73.77631) (end 62.347 59.573) (width 0.2) (layer "B.Cu") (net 2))
 (segment (start 56.759 109.119) (end 56.759 79.36431) (width 0.2) (layer "B.Cu") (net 2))
 (segment (start 60.7 113.06) (end 56.759 109.119) (width 0.2) (layer "B.Cu") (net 2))
 (segment (start 56.759 79.36431) (end 62.347 73.77631) (width 0.2) (layer "B.Cu") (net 2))
 (segment (start 61.280314 114.461) (end 60.119686 114.461) (width 0.2) (layer "B.Cu") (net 17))
 (segment (start 59.807 73.77631) (end 59.807 59.573) (width 0.2) (layer "B.Cu") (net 17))
 (segment (start 59.807 59.573) (end 60.87 58.51) (width 0.2) (layer "B.Cu") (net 17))
 (segment (start 79.75 113.06) (end 62.681314 113.06) (width 0.2) (layer "B.Cu") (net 17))
 (segment (start 60.119686 114.461) (end 56.23031 110.571624) (width 0.2) (layer "B.Cu") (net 17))
 (segment (start 56.23031 110.571624) (end 56.23031 77.353) (width 0.2) (layer "B.Cu") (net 17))
 (segment (start 56.23031 77.353) (end 59.807 73.77631) (width 0.2) (layer "B.Cu") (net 17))
 (segment (start 62.681314 113.06) (end 61.280314 114.461) (width 0.2) (layer "B.Cu") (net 17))
 (segment (start 89.875 58.5) (end 88.774 59.601) (width 0.2) (layer "F.Cu") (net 6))
 (segment (start 78.899 59.601) (end 76.5 62) (width 0.2) (layer "F.Cu") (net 6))
 (segment (start 88.774 59.601) (end 78.899 59.601) (width 0.2) (layer "F.Cu") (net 6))
 (segment (start 89.875 71) (end 89.875 63.75) (width 0.2) (layer "F.Cu") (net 4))
 (segment (start 89.875 63.75) (end 88.125 62) (width 0.2) (layer "F.Cu") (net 4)))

